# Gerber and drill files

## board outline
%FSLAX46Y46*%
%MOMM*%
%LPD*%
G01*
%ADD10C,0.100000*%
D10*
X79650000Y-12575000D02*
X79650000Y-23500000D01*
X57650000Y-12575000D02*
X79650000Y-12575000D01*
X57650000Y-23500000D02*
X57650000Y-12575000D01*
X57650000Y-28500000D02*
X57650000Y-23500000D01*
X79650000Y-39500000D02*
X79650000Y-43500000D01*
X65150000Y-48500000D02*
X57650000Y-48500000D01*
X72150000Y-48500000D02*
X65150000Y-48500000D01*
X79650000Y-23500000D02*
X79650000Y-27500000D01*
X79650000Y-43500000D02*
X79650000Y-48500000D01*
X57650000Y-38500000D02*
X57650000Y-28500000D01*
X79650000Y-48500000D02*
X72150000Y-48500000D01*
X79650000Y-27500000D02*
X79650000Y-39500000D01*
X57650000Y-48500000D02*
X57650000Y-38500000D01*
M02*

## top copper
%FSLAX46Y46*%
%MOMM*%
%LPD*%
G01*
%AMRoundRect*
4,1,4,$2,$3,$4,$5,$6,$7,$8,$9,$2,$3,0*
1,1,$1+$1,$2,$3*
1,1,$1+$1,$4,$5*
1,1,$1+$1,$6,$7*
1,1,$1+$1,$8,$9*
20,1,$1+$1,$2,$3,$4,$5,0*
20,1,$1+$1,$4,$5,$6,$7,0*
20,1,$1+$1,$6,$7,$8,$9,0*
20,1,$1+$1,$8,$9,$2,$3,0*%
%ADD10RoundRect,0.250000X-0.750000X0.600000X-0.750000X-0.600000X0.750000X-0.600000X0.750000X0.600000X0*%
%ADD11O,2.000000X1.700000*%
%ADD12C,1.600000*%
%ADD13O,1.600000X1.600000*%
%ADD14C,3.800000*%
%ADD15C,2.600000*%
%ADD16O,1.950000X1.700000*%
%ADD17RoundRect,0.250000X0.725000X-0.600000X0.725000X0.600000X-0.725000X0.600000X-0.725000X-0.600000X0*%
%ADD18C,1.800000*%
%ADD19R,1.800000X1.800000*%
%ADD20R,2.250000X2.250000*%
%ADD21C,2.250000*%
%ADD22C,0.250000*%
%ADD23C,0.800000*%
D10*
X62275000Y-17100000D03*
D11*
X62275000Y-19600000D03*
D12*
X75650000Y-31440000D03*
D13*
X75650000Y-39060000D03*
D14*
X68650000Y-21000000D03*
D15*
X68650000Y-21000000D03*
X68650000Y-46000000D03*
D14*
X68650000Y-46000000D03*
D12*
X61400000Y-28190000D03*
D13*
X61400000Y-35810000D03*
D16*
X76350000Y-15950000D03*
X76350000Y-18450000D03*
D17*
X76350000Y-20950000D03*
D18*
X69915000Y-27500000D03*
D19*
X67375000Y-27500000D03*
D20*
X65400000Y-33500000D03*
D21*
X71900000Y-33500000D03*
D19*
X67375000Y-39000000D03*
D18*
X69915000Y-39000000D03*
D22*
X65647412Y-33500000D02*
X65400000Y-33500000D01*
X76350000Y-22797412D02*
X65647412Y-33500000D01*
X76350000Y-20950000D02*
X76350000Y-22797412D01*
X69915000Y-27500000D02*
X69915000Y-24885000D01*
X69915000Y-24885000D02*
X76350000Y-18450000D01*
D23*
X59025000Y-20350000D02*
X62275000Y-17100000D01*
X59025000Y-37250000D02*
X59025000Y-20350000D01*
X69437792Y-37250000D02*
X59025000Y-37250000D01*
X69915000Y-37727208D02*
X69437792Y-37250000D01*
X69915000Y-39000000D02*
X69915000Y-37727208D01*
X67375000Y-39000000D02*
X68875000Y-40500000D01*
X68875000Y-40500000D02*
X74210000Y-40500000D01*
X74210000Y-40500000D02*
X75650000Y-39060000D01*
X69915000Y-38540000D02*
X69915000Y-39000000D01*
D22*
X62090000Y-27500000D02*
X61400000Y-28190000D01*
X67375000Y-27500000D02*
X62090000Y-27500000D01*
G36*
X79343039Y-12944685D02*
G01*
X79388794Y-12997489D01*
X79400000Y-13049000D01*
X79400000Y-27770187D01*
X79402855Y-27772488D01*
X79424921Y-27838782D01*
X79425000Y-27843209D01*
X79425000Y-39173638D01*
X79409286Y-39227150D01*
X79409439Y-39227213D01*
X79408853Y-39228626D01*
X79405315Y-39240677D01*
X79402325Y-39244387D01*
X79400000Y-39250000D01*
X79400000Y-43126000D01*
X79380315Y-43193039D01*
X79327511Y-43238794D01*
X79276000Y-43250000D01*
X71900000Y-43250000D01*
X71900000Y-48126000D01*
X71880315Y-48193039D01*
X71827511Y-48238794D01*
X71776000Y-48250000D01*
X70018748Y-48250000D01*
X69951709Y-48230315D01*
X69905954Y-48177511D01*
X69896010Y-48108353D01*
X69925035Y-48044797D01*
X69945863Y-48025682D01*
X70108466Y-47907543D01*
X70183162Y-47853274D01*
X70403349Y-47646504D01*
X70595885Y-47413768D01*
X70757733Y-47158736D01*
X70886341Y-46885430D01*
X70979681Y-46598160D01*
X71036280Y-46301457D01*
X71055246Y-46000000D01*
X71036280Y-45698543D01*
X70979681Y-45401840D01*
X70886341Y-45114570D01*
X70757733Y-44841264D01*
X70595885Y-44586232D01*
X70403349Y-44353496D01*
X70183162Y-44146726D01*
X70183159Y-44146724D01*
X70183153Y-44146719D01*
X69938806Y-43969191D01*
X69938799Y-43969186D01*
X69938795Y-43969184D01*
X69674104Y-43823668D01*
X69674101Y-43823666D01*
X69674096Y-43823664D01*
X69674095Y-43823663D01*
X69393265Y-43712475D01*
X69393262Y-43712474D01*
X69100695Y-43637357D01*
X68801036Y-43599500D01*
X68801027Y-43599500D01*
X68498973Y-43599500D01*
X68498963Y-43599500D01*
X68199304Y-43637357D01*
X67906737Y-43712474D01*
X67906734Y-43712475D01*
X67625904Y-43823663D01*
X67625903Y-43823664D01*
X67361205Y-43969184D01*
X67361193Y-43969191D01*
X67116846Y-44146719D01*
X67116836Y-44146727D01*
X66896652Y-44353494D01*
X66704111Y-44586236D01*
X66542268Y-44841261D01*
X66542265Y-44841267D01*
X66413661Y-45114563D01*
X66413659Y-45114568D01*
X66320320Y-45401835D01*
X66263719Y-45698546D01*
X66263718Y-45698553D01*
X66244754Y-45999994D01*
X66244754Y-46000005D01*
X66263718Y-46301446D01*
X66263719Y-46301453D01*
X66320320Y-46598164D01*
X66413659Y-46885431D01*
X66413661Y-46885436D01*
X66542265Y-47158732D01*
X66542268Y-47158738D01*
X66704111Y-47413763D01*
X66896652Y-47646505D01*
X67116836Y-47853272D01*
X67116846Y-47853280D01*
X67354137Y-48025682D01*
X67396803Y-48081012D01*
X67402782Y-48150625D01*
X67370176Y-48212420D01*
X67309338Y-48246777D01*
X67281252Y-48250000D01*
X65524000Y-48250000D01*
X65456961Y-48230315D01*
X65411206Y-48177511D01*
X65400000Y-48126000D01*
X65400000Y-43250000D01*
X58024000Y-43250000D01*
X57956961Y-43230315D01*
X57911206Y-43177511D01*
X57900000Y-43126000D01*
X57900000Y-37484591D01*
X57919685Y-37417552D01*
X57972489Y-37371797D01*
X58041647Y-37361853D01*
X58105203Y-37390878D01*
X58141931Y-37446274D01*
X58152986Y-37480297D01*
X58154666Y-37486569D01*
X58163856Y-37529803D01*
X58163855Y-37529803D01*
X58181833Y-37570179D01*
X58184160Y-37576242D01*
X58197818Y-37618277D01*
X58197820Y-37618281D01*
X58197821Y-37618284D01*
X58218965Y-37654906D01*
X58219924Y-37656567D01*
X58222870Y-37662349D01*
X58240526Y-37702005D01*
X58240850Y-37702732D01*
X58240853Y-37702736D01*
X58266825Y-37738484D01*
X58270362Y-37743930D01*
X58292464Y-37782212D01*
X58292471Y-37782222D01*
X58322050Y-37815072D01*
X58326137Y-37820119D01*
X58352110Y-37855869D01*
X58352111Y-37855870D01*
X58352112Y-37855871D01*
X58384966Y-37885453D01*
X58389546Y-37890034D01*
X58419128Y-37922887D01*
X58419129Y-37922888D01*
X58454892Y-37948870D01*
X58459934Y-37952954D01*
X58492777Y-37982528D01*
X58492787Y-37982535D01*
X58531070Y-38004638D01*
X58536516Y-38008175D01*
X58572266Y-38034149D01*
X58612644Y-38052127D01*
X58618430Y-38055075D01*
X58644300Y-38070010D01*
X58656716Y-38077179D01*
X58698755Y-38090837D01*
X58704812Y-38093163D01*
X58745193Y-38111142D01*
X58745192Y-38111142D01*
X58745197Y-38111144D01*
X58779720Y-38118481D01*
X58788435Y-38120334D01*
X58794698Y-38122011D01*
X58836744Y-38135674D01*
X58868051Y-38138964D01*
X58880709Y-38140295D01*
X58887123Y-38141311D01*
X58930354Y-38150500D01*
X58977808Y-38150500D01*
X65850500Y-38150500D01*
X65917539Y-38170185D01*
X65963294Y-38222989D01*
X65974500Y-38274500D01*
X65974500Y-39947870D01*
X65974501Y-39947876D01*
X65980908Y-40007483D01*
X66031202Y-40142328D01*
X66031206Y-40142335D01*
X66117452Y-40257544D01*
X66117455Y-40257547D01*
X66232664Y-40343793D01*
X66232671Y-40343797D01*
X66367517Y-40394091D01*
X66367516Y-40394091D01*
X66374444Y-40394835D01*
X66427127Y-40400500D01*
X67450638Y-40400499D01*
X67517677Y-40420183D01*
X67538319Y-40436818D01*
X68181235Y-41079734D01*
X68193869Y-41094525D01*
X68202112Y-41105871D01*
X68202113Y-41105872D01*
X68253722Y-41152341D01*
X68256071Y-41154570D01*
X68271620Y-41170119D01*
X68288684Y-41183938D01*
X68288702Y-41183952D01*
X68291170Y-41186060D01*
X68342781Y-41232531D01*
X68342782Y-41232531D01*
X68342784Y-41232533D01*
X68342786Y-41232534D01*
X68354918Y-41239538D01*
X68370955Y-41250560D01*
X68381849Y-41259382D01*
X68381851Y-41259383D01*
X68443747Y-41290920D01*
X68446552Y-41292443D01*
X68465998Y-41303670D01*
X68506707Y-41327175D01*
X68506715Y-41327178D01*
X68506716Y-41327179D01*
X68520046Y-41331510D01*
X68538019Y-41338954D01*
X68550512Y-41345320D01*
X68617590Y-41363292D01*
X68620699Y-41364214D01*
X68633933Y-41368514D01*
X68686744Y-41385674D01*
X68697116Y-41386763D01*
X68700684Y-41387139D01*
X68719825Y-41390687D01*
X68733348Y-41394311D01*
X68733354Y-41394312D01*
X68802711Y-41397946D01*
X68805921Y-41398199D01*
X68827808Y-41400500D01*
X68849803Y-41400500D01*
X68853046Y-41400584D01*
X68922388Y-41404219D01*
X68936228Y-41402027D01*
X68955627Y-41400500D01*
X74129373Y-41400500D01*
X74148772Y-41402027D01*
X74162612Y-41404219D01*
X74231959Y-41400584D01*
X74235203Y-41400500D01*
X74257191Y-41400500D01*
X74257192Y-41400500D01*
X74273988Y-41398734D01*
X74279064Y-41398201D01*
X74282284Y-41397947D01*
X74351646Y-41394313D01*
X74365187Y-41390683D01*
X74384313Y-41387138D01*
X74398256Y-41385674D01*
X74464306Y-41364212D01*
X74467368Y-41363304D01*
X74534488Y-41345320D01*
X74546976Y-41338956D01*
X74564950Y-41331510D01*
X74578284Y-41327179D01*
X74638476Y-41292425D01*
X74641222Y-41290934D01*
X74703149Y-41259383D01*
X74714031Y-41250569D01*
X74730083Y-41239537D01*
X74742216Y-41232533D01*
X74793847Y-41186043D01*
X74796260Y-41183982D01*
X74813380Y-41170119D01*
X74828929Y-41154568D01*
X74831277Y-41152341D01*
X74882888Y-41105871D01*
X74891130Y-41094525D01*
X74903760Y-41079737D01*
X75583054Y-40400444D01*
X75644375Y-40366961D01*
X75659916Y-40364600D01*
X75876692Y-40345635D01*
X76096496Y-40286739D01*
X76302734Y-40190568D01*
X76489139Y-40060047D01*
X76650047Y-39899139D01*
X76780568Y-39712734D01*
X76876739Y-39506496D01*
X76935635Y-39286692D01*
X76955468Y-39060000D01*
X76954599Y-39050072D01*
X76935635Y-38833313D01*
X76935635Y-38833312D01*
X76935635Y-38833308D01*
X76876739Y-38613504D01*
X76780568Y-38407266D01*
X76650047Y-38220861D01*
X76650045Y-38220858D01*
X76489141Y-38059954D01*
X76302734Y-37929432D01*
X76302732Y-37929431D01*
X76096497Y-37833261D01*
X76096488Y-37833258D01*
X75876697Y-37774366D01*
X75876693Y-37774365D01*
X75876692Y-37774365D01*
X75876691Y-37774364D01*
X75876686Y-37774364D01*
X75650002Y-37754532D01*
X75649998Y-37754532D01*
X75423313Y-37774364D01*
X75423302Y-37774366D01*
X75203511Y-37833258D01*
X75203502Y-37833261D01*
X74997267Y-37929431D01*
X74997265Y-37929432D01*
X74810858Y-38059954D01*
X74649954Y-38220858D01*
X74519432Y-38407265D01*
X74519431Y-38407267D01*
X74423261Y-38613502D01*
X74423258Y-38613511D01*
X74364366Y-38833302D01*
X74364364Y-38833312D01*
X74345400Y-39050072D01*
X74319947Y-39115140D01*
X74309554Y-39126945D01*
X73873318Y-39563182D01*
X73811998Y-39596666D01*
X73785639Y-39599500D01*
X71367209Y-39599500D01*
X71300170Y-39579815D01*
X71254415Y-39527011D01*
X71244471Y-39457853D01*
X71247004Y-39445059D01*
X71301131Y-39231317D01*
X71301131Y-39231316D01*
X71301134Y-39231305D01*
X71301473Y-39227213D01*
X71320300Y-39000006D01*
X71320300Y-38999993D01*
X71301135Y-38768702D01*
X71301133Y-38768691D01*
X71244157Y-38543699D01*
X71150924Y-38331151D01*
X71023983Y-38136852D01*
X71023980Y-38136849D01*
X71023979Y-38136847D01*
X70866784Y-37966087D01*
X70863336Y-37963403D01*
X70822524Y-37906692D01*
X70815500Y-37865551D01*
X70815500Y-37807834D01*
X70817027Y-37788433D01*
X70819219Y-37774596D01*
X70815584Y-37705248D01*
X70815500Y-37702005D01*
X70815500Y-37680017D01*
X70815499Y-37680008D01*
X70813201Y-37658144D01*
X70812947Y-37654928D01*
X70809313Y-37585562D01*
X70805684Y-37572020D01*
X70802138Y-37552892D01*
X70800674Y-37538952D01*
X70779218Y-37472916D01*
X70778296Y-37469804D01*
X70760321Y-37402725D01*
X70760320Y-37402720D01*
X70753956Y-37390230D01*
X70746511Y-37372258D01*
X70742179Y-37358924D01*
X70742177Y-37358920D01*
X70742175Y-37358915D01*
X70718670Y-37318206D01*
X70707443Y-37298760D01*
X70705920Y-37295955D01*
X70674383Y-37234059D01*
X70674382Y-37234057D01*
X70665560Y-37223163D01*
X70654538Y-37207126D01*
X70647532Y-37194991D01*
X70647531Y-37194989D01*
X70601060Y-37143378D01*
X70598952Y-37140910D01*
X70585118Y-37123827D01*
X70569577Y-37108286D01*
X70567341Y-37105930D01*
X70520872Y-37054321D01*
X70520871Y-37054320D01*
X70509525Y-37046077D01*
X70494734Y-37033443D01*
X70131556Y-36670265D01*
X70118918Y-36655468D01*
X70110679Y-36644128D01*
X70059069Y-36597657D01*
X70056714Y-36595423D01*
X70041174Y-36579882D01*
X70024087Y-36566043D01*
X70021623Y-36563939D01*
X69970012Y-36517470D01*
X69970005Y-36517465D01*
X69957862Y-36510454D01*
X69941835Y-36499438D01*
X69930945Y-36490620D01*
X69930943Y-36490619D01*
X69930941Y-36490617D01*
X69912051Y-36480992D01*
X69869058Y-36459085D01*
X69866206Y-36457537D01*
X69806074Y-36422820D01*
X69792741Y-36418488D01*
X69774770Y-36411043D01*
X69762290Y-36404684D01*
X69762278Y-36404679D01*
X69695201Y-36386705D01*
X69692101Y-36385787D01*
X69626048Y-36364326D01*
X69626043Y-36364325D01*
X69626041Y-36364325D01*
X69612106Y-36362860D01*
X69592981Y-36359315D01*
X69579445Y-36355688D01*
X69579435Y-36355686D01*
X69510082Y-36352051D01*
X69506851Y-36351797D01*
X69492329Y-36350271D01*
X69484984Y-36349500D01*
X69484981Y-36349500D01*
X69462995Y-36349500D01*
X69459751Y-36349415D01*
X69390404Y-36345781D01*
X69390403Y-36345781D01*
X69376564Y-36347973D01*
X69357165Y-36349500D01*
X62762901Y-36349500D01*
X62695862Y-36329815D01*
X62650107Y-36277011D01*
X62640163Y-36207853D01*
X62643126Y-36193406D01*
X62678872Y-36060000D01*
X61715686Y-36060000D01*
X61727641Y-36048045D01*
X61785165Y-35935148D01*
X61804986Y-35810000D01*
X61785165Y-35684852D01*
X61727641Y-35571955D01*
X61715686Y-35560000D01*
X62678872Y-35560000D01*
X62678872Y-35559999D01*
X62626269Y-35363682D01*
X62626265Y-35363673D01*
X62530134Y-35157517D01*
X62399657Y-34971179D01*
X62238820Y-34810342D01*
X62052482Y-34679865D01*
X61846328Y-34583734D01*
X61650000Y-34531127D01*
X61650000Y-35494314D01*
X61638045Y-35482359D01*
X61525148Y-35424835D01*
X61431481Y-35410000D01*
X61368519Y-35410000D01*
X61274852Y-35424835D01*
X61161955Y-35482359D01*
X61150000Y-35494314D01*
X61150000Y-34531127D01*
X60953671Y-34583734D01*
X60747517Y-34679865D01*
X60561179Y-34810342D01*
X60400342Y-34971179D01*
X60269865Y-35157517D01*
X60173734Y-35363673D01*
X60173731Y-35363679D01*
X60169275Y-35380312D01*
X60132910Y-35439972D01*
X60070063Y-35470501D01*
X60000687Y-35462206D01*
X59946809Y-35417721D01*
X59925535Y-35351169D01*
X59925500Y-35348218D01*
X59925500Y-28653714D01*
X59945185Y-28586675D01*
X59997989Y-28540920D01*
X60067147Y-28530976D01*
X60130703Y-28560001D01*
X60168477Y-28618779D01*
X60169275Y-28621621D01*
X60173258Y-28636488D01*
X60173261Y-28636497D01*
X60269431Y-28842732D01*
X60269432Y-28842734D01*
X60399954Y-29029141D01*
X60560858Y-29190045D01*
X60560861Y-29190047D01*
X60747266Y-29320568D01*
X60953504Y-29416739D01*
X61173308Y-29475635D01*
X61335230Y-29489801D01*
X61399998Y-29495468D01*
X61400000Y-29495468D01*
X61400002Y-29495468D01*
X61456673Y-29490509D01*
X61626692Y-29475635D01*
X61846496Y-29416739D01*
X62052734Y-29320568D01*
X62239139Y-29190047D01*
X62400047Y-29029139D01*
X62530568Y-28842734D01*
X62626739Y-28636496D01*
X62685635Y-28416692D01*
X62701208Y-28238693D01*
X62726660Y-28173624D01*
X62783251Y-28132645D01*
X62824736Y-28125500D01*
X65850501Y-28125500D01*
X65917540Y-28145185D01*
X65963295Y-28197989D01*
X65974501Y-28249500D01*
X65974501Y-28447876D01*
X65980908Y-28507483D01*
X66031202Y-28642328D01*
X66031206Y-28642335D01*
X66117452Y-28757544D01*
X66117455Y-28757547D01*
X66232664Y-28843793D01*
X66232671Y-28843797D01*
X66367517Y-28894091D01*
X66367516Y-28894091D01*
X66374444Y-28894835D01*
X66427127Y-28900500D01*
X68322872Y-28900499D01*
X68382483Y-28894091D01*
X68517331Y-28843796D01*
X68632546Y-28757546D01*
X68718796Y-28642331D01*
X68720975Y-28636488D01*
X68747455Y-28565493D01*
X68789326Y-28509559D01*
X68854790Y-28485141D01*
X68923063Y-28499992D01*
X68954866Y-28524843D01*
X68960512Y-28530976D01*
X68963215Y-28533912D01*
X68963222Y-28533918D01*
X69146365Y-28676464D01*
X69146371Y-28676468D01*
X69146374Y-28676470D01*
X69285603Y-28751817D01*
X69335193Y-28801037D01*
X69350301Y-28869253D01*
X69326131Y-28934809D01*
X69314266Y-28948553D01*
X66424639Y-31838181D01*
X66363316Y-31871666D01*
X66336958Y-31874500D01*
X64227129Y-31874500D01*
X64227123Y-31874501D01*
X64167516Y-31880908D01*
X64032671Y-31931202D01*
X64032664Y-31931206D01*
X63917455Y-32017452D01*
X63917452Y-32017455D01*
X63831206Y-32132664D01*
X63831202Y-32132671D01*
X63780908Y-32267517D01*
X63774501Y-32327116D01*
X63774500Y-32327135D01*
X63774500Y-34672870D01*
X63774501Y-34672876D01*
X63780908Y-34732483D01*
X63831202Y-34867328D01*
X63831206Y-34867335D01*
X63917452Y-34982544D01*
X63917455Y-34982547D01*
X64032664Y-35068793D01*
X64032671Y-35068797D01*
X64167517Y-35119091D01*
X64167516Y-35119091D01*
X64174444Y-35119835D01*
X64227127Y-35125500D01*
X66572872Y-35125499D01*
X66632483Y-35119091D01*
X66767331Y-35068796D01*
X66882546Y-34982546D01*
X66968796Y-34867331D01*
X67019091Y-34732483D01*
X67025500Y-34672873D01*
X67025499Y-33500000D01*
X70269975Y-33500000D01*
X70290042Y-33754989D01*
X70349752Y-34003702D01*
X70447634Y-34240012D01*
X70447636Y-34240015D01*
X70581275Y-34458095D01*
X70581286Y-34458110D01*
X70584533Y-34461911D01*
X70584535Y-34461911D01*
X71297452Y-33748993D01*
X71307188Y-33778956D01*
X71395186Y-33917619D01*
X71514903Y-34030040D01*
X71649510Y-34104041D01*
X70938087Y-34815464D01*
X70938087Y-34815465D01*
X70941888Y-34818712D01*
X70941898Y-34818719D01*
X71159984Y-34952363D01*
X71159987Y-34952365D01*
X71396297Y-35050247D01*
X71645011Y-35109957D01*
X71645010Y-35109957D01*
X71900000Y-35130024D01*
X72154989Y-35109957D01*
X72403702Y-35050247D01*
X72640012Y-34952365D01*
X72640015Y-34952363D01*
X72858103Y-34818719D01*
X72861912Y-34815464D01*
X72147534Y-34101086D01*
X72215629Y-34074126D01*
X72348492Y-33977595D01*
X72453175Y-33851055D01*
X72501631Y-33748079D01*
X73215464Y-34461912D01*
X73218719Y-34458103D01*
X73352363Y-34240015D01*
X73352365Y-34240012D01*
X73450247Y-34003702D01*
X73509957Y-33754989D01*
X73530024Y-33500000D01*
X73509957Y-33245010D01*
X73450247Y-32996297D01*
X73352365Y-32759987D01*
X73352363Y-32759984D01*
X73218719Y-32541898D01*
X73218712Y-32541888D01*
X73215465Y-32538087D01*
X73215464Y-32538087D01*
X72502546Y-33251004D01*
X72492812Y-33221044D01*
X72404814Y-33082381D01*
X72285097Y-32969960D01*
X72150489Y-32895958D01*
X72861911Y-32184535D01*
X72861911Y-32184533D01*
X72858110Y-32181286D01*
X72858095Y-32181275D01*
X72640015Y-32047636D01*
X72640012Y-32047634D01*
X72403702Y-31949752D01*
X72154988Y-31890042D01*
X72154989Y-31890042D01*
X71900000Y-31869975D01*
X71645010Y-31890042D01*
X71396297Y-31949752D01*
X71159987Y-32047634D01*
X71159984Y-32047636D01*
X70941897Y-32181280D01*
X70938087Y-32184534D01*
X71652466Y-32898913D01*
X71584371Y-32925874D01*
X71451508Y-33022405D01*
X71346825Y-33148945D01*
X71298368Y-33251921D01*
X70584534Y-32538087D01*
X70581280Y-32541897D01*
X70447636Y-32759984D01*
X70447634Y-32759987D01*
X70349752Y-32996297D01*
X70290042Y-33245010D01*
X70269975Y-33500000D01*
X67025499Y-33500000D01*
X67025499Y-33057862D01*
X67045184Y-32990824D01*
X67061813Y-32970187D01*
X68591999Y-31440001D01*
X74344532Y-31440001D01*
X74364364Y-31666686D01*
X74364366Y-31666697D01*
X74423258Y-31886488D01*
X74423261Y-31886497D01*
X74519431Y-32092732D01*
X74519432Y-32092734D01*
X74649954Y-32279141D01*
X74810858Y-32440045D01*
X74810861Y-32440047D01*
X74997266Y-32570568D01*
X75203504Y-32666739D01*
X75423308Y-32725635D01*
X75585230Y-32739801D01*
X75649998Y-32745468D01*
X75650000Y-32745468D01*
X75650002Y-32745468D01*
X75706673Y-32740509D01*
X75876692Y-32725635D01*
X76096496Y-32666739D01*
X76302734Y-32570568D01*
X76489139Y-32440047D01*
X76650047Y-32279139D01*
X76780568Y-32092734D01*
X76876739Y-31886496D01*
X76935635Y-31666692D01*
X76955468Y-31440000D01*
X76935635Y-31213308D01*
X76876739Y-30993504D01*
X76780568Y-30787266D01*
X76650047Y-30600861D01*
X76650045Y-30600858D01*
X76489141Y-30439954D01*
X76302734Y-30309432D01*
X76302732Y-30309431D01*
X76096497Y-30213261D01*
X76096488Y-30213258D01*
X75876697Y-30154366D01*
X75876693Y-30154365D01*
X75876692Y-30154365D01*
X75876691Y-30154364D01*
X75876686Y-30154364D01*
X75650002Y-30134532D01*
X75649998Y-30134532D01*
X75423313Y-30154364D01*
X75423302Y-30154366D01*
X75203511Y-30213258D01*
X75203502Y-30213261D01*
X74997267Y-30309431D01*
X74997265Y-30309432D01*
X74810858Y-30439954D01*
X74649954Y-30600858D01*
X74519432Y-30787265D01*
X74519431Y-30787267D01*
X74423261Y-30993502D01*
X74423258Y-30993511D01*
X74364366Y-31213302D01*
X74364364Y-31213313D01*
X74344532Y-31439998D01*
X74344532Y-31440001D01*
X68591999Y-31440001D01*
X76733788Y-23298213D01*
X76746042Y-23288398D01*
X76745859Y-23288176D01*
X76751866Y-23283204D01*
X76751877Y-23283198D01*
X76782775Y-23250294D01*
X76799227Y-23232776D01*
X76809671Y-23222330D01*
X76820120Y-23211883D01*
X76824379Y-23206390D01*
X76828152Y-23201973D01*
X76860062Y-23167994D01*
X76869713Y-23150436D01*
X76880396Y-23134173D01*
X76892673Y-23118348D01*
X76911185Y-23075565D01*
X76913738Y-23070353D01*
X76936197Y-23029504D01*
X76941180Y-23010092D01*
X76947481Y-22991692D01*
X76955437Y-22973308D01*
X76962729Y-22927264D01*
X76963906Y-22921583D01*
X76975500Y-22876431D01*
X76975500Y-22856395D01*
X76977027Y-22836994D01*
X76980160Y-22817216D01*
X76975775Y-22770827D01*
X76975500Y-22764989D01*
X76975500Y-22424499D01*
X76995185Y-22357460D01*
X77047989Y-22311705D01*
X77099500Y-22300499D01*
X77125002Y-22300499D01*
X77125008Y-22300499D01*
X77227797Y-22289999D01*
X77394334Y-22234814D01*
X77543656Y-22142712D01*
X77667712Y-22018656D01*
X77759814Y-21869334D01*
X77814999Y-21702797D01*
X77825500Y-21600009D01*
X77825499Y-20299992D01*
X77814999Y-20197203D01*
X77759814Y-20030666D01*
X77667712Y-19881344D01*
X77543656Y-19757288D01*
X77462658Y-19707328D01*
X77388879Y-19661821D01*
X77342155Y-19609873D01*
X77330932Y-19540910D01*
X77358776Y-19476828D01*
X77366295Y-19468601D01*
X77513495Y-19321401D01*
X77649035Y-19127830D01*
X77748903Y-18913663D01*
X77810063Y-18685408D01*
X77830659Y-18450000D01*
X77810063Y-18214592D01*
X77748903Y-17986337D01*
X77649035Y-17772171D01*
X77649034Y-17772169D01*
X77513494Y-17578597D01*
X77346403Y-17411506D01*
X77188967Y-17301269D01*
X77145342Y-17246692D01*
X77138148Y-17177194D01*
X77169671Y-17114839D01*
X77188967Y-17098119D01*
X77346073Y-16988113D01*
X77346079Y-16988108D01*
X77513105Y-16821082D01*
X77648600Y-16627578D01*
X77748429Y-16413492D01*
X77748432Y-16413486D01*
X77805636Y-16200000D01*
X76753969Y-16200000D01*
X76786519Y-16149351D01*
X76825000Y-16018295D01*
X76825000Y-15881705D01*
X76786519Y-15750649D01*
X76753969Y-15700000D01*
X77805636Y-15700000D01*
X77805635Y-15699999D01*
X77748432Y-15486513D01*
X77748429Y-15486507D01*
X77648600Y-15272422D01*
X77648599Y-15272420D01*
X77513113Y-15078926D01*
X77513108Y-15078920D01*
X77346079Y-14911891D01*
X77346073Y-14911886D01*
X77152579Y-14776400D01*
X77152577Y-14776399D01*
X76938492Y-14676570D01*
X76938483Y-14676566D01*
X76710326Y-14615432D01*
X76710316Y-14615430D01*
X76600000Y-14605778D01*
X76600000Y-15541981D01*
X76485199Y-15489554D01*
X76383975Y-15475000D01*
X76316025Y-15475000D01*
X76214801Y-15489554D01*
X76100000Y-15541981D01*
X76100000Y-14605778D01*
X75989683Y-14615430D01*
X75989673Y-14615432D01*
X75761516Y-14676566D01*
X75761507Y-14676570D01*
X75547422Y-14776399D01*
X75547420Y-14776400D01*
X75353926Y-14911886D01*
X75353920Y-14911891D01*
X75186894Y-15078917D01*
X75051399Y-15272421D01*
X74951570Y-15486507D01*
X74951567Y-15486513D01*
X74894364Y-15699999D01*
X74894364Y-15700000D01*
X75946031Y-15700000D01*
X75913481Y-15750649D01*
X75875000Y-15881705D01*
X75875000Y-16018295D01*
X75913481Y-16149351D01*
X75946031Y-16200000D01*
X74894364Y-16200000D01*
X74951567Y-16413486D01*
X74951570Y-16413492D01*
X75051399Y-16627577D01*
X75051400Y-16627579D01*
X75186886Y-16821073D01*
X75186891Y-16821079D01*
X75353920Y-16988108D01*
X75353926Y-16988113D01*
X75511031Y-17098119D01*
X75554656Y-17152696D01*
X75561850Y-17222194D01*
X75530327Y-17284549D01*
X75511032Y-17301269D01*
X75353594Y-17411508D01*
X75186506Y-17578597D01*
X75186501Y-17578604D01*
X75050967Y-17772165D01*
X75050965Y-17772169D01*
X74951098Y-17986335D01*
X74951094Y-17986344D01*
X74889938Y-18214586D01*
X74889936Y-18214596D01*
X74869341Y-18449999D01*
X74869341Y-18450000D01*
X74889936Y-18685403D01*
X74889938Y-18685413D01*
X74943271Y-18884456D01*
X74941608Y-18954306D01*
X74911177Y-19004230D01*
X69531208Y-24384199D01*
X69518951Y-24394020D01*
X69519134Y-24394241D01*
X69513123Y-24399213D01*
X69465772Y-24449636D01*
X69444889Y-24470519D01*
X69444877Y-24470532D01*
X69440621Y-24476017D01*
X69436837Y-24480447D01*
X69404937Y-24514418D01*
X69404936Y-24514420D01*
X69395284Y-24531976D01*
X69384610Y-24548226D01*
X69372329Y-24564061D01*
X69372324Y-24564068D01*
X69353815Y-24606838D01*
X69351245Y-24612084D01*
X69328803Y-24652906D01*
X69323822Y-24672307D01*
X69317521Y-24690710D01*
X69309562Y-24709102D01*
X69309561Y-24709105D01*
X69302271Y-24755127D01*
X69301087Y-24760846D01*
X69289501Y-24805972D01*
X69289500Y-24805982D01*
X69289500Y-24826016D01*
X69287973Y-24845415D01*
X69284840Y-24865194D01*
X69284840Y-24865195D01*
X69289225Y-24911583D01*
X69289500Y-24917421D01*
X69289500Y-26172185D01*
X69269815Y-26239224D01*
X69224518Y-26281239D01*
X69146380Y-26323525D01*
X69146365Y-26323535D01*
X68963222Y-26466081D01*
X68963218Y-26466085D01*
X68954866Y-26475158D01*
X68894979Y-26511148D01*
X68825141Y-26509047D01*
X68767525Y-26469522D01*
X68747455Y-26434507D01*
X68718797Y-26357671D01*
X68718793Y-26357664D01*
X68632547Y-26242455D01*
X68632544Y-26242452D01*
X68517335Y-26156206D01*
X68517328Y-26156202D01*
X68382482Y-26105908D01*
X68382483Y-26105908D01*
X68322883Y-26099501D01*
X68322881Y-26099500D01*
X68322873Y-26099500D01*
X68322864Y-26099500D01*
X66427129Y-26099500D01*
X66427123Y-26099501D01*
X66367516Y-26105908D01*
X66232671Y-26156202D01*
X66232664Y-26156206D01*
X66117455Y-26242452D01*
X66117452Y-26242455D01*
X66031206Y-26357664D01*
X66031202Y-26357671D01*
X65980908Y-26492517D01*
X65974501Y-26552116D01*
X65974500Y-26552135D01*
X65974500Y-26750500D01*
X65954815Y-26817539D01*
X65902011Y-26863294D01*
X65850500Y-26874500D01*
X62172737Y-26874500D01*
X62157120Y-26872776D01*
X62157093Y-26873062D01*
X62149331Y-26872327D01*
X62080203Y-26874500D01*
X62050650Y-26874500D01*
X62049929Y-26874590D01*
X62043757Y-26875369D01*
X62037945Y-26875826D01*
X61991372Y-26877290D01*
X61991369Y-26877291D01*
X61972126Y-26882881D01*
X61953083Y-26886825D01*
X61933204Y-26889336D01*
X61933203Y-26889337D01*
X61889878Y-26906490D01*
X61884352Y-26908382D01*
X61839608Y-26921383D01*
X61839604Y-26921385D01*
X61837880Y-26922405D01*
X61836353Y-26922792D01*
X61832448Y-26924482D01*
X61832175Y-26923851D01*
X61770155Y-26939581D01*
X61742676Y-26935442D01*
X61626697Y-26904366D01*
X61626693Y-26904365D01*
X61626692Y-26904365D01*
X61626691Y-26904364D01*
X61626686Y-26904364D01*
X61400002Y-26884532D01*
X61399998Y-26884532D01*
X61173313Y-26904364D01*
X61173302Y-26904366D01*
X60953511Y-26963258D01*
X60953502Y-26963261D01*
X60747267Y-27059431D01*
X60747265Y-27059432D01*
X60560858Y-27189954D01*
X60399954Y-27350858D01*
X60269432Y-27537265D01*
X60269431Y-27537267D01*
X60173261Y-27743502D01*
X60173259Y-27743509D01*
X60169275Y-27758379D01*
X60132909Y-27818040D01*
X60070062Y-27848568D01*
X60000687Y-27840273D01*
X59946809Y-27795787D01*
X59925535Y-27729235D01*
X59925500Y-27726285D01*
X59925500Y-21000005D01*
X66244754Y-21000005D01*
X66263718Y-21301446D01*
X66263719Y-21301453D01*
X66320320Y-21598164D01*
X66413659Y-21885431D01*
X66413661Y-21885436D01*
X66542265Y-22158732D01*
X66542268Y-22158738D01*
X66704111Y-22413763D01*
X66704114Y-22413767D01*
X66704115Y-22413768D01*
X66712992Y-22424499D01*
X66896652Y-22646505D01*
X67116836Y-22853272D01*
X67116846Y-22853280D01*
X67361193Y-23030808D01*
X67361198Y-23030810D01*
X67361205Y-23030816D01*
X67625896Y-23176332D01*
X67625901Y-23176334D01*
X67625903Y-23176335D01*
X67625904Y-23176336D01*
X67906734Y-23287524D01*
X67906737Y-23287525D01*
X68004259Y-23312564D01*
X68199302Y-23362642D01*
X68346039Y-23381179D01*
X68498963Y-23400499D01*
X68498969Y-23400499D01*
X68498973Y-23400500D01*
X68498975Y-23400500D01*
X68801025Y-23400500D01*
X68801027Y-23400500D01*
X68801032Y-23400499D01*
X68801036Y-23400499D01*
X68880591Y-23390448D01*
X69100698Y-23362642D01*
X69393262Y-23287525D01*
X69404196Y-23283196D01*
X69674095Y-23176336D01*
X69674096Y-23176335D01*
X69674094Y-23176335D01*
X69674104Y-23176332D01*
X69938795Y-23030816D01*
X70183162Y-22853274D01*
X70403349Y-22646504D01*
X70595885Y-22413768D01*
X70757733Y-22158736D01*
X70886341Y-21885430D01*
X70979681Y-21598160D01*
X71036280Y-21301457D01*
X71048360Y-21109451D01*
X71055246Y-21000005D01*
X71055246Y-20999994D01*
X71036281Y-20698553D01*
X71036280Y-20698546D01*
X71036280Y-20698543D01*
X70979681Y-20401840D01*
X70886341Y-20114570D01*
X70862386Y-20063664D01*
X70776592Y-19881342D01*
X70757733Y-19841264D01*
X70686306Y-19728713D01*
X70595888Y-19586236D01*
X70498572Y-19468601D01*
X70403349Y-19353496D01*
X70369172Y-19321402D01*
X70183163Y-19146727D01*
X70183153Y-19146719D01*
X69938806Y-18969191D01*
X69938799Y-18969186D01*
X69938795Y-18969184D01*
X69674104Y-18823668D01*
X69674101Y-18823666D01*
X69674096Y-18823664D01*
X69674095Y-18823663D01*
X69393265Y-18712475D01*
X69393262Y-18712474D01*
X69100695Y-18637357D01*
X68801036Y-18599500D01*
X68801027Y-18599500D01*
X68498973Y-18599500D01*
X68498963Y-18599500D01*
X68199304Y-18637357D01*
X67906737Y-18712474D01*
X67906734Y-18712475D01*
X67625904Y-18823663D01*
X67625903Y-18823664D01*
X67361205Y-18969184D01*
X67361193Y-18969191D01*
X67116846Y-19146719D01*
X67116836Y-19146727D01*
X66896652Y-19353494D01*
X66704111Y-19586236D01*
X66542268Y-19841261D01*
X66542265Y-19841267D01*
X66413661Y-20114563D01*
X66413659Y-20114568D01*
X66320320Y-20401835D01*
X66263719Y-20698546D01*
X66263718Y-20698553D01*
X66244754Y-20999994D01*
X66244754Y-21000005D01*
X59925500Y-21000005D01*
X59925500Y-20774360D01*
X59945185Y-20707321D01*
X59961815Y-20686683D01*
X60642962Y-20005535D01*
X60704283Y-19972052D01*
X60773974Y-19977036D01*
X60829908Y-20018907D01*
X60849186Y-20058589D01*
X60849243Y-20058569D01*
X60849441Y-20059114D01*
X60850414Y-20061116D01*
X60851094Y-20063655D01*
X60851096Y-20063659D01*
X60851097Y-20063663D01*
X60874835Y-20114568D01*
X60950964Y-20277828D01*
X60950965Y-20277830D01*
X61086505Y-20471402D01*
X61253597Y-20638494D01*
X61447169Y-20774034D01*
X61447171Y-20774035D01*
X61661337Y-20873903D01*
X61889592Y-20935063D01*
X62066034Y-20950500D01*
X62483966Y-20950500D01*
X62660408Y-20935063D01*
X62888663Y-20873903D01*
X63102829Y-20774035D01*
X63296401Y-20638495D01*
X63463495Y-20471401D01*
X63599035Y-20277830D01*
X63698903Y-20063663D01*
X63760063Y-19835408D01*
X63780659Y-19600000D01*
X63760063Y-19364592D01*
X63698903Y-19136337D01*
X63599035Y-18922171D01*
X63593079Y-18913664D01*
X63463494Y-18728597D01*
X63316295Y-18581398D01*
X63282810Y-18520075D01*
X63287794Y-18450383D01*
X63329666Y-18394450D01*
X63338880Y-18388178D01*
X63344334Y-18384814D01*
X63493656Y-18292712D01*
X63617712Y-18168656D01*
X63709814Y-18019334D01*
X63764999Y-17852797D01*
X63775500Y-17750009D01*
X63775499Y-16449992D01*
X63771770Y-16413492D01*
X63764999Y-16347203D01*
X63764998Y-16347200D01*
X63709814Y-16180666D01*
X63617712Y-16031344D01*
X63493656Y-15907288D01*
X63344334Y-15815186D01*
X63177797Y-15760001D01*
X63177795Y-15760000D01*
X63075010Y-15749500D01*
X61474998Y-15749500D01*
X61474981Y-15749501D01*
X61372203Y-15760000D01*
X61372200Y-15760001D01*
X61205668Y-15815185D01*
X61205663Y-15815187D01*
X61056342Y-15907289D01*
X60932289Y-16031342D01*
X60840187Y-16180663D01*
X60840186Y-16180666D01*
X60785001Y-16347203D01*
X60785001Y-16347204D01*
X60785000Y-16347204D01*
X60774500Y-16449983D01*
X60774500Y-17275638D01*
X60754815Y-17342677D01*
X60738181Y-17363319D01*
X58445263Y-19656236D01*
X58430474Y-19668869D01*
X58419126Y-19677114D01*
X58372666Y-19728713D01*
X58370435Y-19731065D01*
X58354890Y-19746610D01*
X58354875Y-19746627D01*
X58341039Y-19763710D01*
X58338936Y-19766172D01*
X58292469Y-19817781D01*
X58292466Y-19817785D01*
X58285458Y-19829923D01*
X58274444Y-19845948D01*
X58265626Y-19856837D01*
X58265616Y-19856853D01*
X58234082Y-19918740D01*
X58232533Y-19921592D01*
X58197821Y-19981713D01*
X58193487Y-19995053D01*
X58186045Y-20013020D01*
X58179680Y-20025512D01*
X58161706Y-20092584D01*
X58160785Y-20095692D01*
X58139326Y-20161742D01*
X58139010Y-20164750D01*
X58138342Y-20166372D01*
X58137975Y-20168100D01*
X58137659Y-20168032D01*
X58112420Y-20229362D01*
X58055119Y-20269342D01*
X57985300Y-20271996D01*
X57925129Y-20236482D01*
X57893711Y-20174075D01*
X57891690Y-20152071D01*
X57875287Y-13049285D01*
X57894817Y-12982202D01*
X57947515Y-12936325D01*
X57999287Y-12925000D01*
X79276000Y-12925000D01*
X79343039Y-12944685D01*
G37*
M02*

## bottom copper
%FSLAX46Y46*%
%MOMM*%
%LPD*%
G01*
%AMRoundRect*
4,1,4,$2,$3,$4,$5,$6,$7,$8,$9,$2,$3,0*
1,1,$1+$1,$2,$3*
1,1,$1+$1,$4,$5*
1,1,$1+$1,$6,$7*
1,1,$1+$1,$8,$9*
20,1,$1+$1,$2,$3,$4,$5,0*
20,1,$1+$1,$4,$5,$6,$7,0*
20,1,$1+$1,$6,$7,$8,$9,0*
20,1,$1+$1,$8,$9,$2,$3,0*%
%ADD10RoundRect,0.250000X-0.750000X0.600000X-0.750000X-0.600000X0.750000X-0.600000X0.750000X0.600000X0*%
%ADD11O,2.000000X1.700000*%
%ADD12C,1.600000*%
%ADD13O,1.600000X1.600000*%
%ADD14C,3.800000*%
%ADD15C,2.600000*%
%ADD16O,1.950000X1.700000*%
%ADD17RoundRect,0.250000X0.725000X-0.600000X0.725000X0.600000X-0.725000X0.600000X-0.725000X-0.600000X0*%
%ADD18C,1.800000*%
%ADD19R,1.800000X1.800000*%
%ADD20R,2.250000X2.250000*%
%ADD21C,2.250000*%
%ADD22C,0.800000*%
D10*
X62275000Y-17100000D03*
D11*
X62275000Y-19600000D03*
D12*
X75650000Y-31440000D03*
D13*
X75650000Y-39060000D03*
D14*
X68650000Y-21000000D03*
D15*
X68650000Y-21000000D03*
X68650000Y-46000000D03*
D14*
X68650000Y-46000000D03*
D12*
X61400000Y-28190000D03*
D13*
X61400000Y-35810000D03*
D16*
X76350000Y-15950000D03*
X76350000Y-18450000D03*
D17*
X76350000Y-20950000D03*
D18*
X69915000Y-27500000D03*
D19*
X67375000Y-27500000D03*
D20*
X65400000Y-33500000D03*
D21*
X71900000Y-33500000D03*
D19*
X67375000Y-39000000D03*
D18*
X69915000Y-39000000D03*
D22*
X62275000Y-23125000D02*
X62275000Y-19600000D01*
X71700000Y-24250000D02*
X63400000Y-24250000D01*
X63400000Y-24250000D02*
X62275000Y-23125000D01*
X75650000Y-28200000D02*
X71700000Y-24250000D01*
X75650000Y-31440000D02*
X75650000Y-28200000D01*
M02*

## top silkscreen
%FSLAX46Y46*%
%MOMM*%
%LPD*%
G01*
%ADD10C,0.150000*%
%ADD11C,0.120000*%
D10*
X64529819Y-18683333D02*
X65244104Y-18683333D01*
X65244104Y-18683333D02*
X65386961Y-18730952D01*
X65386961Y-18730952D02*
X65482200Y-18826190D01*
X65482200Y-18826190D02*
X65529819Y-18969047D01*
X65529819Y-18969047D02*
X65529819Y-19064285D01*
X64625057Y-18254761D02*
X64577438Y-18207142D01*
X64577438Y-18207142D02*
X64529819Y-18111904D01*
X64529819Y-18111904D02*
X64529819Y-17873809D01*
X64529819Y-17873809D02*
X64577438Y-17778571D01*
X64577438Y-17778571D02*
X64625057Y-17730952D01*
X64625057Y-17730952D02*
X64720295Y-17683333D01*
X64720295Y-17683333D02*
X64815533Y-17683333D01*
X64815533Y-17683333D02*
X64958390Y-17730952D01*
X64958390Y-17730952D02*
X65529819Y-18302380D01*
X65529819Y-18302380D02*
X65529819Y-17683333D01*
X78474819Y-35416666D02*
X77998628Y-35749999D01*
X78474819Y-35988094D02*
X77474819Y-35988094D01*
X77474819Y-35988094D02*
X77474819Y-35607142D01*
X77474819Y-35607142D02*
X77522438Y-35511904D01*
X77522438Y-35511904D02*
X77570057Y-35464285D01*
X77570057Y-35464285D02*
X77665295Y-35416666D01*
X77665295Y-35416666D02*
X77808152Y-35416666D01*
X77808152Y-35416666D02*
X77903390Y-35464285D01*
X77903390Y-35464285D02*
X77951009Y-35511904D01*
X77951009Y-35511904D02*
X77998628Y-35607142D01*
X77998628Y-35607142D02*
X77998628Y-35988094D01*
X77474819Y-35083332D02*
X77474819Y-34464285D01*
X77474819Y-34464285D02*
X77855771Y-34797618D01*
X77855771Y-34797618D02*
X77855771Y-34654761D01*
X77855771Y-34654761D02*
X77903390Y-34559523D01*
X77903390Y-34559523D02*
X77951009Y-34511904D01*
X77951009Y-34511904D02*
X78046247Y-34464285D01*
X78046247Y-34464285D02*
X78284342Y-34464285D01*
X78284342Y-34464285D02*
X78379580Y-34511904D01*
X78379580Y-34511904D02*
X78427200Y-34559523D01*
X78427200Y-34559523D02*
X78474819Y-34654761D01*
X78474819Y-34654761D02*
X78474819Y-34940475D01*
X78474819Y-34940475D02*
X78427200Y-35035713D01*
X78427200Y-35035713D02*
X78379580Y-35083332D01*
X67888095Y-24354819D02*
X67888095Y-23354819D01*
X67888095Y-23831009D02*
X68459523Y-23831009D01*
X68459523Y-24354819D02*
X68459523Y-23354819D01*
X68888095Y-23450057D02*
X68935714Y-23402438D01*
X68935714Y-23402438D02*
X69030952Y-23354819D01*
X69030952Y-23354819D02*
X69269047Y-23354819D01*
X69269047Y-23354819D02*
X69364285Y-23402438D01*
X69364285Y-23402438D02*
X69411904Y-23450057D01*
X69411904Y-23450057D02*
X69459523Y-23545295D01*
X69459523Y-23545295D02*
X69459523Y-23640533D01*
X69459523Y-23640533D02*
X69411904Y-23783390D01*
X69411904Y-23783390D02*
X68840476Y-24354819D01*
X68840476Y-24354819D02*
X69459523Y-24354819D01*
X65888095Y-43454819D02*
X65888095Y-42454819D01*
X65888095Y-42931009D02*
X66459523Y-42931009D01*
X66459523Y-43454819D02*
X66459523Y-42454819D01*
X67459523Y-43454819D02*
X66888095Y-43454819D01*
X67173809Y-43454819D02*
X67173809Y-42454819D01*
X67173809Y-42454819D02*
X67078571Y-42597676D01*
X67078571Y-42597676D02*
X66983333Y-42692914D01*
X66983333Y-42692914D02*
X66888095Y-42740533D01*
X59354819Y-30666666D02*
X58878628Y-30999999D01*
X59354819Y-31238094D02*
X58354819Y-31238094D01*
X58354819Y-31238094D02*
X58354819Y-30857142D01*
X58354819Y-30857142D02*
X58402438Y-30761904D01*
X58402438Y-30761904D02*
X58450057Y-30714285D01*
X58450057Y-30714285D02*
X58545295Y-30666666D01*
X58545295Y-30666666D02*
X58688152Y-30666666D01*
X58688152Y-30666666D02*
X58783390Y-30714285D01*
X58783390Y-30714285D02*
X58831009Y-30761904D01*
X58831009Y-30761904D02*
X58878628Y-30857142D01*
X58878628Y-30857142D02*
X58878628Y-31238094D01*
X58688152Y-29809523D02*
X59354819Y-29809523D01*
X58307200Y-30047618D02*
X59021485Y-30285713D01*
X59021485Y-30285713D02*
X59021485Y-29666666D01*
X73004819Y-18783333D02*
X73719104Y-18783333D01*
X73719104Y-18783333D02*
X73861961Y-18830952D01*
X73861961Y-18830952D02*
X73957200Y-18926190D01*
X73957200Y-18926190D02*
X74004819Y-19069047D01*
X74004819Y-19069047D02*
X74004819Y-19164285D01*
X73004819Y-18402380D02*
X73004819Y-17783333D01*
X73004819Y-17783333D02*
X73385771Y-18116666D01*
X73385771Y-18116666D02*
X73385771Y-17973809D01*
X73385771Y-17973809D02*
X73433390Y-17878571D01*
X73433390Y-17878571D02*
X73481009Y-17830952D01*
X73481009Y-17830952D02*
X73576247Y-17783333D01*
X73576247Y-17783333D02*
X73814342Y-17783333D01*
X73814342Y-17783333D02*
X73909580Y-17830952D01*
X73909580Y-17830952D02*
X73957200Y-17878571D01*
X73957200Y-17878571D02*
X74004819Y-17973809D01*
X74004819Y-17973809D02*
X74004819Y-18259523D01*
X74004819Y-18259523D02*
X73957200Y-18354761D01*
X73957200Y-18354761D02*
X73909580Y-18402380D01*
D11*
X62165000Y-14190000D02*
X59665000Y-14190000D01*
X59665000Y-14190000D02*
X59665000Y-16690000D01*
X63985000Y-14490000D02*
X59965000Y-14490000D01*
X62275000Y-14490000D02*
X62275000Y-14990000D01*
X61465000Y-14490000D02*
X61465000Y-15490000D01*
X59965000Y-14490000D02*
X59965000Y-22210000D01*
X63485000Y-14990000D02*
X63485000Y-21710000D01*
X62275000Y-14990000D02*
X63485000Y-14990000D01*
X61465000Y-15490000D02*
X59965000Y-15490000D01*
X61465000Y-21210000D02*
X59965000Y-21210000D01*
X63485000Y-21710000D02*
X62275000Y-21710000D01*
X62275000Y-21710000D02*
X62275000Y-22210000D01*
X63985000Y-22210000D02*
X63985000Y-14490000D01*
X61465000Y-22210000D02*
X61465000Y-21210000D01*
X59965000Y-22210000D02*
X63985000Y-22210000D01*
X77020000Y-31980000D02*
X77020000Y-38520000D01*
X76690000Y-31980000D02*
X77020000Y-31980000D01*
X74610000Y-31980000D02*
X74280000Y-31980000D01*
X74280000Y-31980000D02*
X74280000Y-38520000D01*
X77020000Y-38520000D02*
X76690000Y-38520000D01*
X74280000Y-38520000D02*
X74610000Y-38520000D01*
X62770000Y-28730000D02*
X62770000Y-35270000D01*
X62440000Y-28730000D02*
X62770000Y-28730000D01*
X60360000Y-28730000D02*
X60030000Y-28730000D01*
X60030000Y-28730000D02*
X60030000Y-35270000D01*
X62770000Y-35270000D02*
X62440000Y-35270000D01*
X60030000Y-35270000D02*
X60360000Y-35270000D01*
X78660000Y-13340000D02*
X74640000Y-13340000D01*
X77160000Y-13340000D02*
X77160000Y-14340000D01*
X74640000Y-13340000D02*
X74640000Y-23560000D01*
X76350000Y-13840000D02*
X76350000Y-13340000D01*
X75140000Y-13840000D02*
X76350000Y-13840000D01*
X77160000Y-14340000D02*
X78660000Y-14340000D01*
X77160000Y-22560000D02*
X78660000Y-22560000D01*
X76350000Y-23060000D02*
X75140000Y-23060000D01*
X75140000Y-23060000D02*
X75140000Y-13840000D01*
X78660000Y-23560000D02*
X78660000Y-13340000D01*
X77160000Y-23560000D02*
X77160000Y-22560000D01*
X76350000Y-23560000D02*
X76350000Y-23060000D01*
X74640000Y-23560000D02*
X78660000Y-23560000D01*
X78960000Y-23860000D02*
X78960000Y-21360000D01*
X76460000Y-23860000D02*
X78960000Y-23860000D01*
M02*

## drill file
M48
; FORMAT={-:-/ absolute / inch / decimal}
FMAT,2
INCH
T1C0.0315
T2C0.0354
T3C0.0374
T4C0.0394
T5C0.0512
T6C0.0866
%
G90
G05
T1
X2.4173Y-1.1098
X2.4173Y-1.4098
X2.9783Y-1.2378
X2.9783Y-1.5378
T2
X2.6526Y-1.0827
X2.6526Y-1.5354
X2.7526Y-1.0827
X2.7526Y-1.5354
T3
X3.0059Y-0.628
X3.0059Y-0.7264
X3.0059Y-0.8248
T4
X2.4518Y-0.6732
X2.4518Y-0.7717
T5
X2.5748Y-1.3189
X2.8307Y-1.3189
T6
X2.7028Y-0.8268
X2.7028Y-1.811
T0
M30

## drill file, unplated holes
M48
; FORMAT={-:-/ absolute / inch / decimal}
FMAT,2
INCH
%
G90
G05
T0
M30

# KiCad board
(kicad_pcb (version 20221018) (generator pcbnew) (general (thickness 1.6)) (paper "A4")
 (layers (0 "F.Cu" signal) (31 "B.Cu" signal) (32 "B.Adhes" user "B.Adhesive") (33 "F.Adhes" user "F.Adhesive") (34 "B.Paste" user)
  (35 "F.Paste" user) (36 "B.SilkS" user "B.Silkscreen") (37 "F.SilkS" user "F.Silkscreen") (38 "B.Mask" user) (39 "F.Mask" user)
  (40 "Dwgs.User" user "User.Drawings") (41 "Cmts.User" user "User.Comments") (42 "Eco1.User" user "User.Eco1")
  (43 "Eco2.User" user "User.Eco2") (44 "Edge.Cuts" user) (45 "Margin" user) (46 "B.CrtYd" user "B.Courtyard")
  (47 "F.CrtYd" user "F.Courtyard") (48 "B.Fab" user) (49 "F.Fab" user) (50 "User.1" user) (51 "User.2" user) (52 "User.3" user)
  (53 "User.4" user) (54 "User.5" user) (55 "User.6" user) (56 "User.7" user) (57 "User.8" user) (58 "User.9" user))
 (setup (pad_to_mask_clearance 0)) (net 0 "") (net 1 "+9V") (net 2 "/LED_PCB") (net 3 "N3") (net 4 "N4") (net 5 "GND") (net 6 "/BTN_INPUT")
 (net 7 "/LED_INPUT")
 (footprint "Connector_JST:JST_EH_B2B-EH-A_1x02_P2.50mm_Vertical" (layer "F.Cu") (at 62.275 17.1 -90)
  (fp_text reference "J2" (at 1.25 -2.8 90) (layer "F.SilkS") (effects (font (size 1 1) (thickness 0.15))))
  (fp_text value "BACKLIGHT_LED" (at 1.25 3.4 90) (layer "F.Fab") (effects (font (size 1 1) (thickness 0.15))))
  (fp_line (start -2.91 0.11) (end -2.91 2.61) (stroke (width 0.12) (type solid)) (layer "F.SilkS"))
  (fp_line (start -2.91 2.61) (end -0.41 2.61) (stroke (width 0.12) (type solid)) (layer "F.SilkS"))
  (fp_line (start -2.61 -1.71) (end -2.61 2.31) (stroke (width 0.12) (type solid)) (layer "F.SilkS"))
  (fp_line (start -2.61 0) (end -2.11 0) (stroke (width 0.12) (type solid)) (layer "F.SilkS"))
  (fp_line (start -2.61 0.81) (end -1.61 0.81) (stroke (width 0.12) (type solid)) (layer "F.SilkS"))
  (fp_line (start -2.61 2.31) (end 5.11 2.31) (stroke (width 0.12) (type solid)) (layer "F.SilkS"))
  (fp_line (start -2.11 -1.21) (end 4.61 -1.21) (stroke (width 0.12) (type solid)) (layer "F.SilkS"))
  (fp_line (start -2.11 0) (end -2.11 -1.21) (stroke (width 0.12) (type solid)) (layer "F.SilkS"))
  (fp_line (start -1.61 0.81) (end -1.61 2.31) (stroke (width 0.12) (type solid)) (layer "F.SilkS"))
  (fp_line (start 4.11 0.81) (end 4.11 2.31) (stroke (width 0.12) (type solid)) (layer "F.SilkS"))
  (fp_line (start 4.61 -1.21) (end 4.61 0) (stroke (width 0.12) (type solid)) (layer "F.SilkS"))
  (fp_line (start 4.61 0) (end 5.11 0) (stroke (width 0.12) (type solid)) (layer "F.SilkS"))
  (fp_line (start 5.11 -1.71) (end -2.61 -1.71) (stroke (width 0.12) (type solid)) (layer "F.SilkS"))
  (fp_line (start 5.11 0.81) (end 4.11 0.81) (stroke (width 0.12) (type solid)) (layer "F.SilkS"))
  (fp_line (start 5.11 2.31) (end 5.11 -1.71) (stroke (width 0.12) (type solid)) (layer "F.SilkS"))
  (pad "1" thru_hole roundrect (at 0 0 270) (size 1.7 2) (drill 1) (layers "*.Cu" "*.Mask") (roundrect_rratio 0.147059) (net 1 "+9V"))
  (pad "2" thru_hole oval (at 2.5 0 270) (size 1.7 2) (drill 1) (layers "*.Cu" "*.Mask") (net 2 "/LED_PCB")))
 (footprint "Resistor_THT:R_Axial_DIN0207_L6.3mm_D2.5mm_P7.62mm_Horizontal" (layer "F.Cu") (at 75.65 31.44 -90)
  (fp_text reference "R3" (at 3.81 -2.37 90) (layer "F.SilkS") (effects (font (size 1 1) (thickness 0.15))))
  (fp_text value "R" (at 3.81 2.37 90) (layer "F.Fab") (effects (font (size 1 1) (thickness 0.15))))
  (fp_line (start 0.54 -1.37) (end 7.08 -1.37) (stroke (width 0.12) (type solid)) (layer "F.SilkS"))
  (fp_line (start 0.54 -1.04) (end 0.54 -1.37) (stroke (width 0.12) (type solid)) (layer "F.SilkS"))
  (fp_line (start 0.54 1.04) (end 0.54 1.37) (stroke (width 0.12) (type solid)) (layer "F.SilkS"))
  (fp_line (start 0.54 1.37) (end 7.08 1.37) (stroke (width 0.12) (type solid)) (layer "F.SilkS"))
  (fp_line (start 7.08 -1.37) (end 7.08 -1.04) (stroke (width 0.12) (type solid)) (layer "F.SilkS"))
  (fp_line (start 7.08 1.37) (end 7.08 1.04) (stroke (width 0.12) (type solid)) (layer "F.SilkS"))
  (pad "1" thru_hole circle (at 0 0 270) (size 1.6 1.6) (drill 0.8) (layers "*.Cu" "*.Mask") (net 2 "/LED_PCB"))
  (pad "2" thru_hole oval (at 7.62 0 270) (size 1.6 1.6) (drill 0.8) (layers "*.Cu" "*.Mask") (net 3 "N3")))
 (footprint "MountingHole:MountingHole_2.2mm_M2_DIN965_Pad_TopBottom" (layer "F.Cu") (at 68.65 21 180)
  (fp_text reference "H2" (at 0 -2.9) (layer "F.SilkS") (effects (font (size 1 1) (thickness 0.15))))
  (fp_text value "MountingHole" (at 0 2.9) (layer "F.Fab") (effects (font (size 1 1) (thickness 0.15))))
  (pad "1" thru_hole circle (at 0 0 180) (size 2.6 2.6) (drill 2.2) (layers "*.Cu" "*.Mask"))
  (pad "1" connect circle (at 0 0 180) (size 3.8 3.8) (layers "F.Cu" "F.Mask"))
  (pad "1" connect circle (at 0 0 180) (size 3.8 3.8) (layers "B.Cu" "B.Mask")))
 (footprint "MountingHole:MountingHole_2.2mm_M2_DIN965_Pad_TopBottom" (layer "F.Cu") (at 68.65 46 180)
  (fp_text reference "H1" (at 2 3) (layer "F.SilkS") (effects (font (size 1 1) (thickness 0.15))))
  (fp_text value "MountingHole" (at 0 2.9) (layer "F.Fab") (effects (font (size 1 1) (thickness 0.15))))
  (pad "1" thru_hole circle (at 0 0 180) (size 2.6 2.6) (drill 2.2) (layers "*.Cu" "*.Mask"))
  (pad "1" connect circle (at 0 0 180) (size 3.8 3.8) (layers "F.Cu" "F.Mask"))
  (pad "1" connect circle (at 0 0 180) (size 3.8 3.8) (layers "B.Cu" "B.Mask")))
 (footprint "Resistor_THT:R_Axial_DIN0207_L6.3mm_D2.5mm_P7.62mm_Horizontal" (layer "F.Cu") (at 61.4 28.19 -90)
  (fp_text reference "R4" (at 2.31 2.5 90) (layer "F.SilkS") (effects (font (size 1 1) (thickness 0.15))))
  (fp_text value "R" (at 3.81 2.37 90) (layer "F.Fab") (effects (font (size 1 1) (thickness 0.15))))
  (fp_line (start 0.54 -1.37) (end 7.08 -1.37) (stroke (width 0.12) (type solid)) (layer "F.SilkS"))
  (fp_line (start 0.54 -1.04) (end 0.54 -1.37) (stroke (width 0.12) (type solid)) (layer "F.SilkS"))
  (fp_line (start 0.54 1.04) (end 0.54 1.37) (stroke (width 0.12) (type solid)) (layer "F.SilkS"))
  (fp_line (start 0.54 1.37) (end 7.08 1.37) (stroke (width 0.12) (type solid)) (layer "F.SilkS"))
  (fp_line (start 7.08 -1.37) (end 7.08 -1.04) (stroke (width 0.12) (type solid)) (layer "F.SilkS"))
  (fp_line (start 7.08 1.37) (end 7.08 1.04) (stroke (width 0.12) (type solid)) (layer "F.SilkS"))
  (pad "1" thru_hole circle (at 0 0 270) (size 1.6 1.6) (drill 0.8) (layers "*.Cu" "*.Mask") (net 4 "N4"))
  (pad "2" thru_hole oval (at 7.62 0 270) (size 1.6 1.6) (drill 0.8) (layers "*.Cu" "*.Mask") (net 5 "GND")))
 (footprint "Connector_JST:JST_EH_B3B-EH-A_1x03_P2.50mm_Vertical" (layer "F.Cu") (at 76.35 20.95 90)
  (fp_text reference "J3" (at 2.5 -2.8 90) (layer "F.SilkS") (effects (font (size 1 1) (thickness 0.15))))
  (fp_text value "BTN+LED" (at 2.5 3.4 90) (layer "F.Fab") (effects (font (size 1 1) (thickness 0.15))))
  (fp_line (start -2.91 0.11) (end -2.91 2.61) (stroke (width 0.12) (type solid)) (layer "F.SilkS"))
  (fp_line (start -2.91 2.61) (end -0.41 2.61) (stroke (width 0.12) (type solid)) (layer "F.SilkS"))
  (fp_line (start -2.61 -1.71) (end -2.61 2.31) (stroke (width 0.12) (type solid)) (layer "F.SilkS"))
  (fp_line (start -2.61 0) (end -2.11 0) (stroke (width 0.12) (type solid)) (layer "F.SilkS"))
  (fp_line (start -2.61 0.81) (end -1.61 0.81) (stroke (width 0.12) (type solid)) (layer "F.SilkS"))
  (fp_line (start -2.61 2.31) (end 7.61 2.31) (stroke (width 0.12) (type solid)) (layer "F.SilkS"))
  (fp_line (start -2.11 -1.21) (end 7.11 -1.21) (stroke (width 0.12) (type solid)) (layer "F.SilkS"))
  (fp_line (start -2.11 0) (end -2.11 -1.21) (stroke (width 0.12) (type solid)) (layer "F.SilkS"))
  (fp_line (start -1.61 0.81) (end -1.61 2.31) (stroke (width 0.12) (type solid)) (layer "F.SilkS"))
  (fp_line (start 6.61 0.81) (end 6.61 2.31) (stroke (width 0.12) (type solid)) (layer "F.SilkS"))
  (fp_line (start 7.11 -1.21) (end 7.11 0) (stroke (width 0.12) (type solid)) (layer "F.SilkS"))
  (fp_line (start 7.11 0) (end 7.61 0) (stroke (width 0.12) (type solid)) (layer "F.SilkS"))
  (fp_line (start 7.61 -1.71) (end -2.61 -1.71) (stroke (width 0.12) (type solid)) (layer "F.SilkS"))
  (fp_line (start 7.61 0.81) (end 6.61 0.81) (stroke (width 0.12) (type solid)) (layer "F.SilkS"))
  (fp_line (start 7.61 2.31) (end 7.61 -1.71) (stroke (width 0.12) (type solid)) (layer "F.SilkS"))
  (pad "1" thru_hole roundrect (at 0 0 90) (size 1.7 1.95) (drill 0.95) (layers "*.Cu" "*.Mask") (roundrect_rratio 0.147059)
   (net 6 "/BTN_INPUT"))
  (pad "2" thru_hole oval (at 2.5 0 90) (size 1.7 1.95) (drill 0.95) (layers "*.Cu" "*.Mask") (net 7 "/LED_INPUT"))
  (pad "3" thru_hole oval (at 5 0 90) (size 1.7 1.95) (drill 0.95) (layers "*.Cu" "*.Mask") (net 5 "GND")))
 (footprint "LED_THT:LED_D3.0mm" (layer "B.Cu") (at 67.375 27.5)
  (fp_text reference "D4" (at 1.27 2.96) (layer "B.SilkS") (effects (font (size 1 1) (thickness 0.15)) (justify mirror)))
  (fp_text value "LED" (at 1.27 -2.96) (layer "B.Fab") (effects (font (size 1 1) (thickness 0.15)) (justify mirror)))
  (pad "1" thru_hole rect (at 0 0) (size 1.8 1.8) (drill 0.9) (layers "*.Cu" "*.Mask") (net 4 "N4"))
  (pad "2" thru_hole circle (at 2.54 0) (size 1.8 1.8) (drill 0.9) (layers "*.Cu" "*.Mask") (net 7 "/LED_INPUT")))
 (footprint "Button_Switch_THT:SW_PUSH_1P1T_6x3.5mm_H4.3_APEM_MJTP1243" (layer "B.Cu") (at 65.4 33.5)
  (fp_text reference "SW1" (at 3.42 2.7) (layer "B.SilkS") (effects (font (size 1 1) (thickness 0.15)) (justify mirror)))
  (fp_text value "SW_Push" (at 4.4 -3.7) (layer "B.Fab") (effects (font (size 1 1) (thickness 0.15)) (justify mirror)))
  (pad "1" thru_hole rect (at 0 0 270) (size 2.25 2.25) (drill 1.3) (layers "*.Cu" "*.Mask") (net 6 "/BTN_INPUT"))
  (pad "2" thru_hole circle (at 6.5 0 270) (size 2.25 2.25) (drill 1.3) (layers "*.Cu" "*.Mask") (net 5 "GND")))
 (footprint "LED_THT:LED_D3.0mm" (layer "B.Cu") (at 67.375 39)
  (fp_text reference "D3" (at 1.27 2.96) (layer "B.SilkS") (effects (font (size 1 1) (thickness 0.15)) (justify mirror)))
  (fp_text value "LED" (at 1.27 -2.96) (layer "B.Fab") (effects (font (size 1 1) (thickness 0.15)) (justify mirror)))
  (pad "1" thru_hole rect (at 0 0) (size 1.8 1.8) (drill 0.9) (layers "*.Cu" "*.Mask") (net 3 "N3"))
  (pad "2" thru_hole circle (at 2.54 0) (size 1.8 1.8) (drill 0.9) (layers "*.Cu" "*.Mask") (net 1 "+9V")))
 (gr_line (start 57.65 28.5) (end 57.65 23.5) (stroke (width 0.1) (type default)) (layer "Edge.Cuts"))
 (gr_line (start 79.65 39.5) (end 79.65 43.5) (stroke (width 0.1) (type default)) (layer "Edge.Cuts"))
 (gr_line (start 65.15 48.5) (end 57.65 48.5) (stroke (width 0.1) (type default)) (layer "Edge.Cuts"))
 (gr_line (start 79.65 12.575) (end 79.65 23.5) (stroke (width 0.1) (type default)) (layer "Edge.Cuts"))
 (gr_line (start 72.15 48.5) (end 65.15 48.5) (stroke (width 0.1) (type default)) (layer "Edge.Cuts"))
 (gr_line (start 79.65 23.5) (end 79.65 27.5) (stroke (width 0.1) (type default)) (layer "Edge.Cuts"))
 (gr_line (start 79.65 43.5) (end 79.65 48.5) (stroke (width 0.1) (type default)) (layer "Edge.Cuts"))
 (gr_line (start 57.65 38.5) (end 57.65 28.5) (stroke (width 0.1) (type default)) (layer "Edge.Cuts"))
 (gr_line (start 79.65 48.5) (end 72.15 48.5) (stroke (width 0.1) (type default)) (layer "Edge.Cuts"))
 (gr_line (start 79.65 27.5) (end 79.65 39.5) (stroke (width 0.1) (type default)) (layer "Edge.Cuts"))
 (gr_line (start 57.65 12.575) (end 79.65 12.575) (stroke (width 0.1) (type default)) (layer "Edge.Cuts"))
 (gr_line (start 57.65 48.5) (end 57.65 38.5) (stroke (width 0.1) (type default)) (layer "Edge.Cuts"))
 (gr_line (start 57.65 23.5) (end 57.65 12.575) (stroke (width 0.1) (type default)) (layer "Edge.Cuts"))
 (segment (start 67.375 39) (end 68.875 40.5) (width 0.8) (layer "F.Cu") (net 3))
 (segment (start 68.875 40.5) (end 74.21 40.5) (width 0.8) (layer "F.Cu") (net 3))
 (segment (start 74.21 40.5) (end 75.65 39.06) (width 0.8) (layer "F.Cu") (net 3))
 (segment (start 59.025 20.35) (end 62.275 17.1) (width 0.8) (layer "F.Cu") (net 1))
 (segment (start 69.437792 37.25) (end 59.025 37.25) (width 0.8) (layer "F.Cu") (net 1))
 (segment (start 69.915 37.727208) (end 69.437792 37.25) (width 0.8) (layer "F.Cu") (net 1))
 (segment (start 69.915 38.54) (end 69.915 39) (width 0.8) (layer "F.Cu") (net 1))
 (segment (start 69.915 39) (end 69.915 37.727208) (width 0.8) (layer "F.Cu") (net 1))
 (segment (start 59.025 37.25) (end 59.025 20.35) (width 0.8) (layer "F.Cu") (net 1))
 (segment (start 62.09 27.5) (end 61.4 28.19) (width 0.25) (layer "F.Cu") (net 4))
 (segment (start 67.375 27.5) (end 62.09 27.5) (width 0.25) (layer "F.Cu") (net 4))
 (segment (start 69.915 24.885) (end 76.35 18.45) (width 0.25) (layer "F.Cu") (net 7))
 (segment (start 69.915 27.5) (end 69.915 24.885) (width 0.25) (layer "F.Cu") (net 7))
 (segment (start 76.35 20.95) (end 76.35 22.797412) (width 0.25) (layer "F.Cu") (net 6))
 (segment (start 76.35 22.797412) (end 65.647412 33.5) (width 0.25) (layer "F.Cu") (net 6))
 (segment (start 65.647412 33.5) (end 65.4 33.5) (width 0.25) (layer "F.Cu") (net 6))
 (segment (start 63.4 24.25) (end 62.275 23.125) (width 0.8) (layer "B.Cu") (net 2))
 (segment (start 71.7 24.25) (end 63.4 24.25) (width 0.8) (layer "B.Cu") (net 2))
 (segment (start 75.65 31.44) (end 75.65 28.2) (width 0.8) (layer "B.Cu") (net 2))
 (segment (start 75.65 28.2) (end 71.7 24.25) (width 0.8) (layer "B.Cu") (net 2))
 (segment (start 62.275 23.125) (end 62.275 19.6) (width 0.8) (layer "B.Cu") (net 2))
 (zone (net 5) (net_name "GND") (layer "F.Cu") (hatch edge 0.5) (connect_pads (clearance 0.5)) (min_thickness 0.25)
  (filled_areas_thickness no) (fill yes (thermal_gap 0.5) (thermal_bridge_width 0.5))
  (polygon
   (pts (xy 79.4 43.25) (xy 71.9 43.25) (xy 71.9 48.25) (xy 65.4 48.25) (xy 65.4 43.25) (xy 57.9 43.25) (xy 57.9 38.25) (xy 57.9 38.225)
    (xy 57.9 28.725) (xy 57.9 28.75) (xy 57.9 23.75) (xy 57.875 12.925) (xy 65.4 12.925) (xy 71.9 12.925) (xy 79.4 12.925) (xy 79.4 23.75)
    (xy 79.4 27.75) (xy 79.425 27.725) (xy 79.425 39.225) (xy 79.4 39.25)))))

